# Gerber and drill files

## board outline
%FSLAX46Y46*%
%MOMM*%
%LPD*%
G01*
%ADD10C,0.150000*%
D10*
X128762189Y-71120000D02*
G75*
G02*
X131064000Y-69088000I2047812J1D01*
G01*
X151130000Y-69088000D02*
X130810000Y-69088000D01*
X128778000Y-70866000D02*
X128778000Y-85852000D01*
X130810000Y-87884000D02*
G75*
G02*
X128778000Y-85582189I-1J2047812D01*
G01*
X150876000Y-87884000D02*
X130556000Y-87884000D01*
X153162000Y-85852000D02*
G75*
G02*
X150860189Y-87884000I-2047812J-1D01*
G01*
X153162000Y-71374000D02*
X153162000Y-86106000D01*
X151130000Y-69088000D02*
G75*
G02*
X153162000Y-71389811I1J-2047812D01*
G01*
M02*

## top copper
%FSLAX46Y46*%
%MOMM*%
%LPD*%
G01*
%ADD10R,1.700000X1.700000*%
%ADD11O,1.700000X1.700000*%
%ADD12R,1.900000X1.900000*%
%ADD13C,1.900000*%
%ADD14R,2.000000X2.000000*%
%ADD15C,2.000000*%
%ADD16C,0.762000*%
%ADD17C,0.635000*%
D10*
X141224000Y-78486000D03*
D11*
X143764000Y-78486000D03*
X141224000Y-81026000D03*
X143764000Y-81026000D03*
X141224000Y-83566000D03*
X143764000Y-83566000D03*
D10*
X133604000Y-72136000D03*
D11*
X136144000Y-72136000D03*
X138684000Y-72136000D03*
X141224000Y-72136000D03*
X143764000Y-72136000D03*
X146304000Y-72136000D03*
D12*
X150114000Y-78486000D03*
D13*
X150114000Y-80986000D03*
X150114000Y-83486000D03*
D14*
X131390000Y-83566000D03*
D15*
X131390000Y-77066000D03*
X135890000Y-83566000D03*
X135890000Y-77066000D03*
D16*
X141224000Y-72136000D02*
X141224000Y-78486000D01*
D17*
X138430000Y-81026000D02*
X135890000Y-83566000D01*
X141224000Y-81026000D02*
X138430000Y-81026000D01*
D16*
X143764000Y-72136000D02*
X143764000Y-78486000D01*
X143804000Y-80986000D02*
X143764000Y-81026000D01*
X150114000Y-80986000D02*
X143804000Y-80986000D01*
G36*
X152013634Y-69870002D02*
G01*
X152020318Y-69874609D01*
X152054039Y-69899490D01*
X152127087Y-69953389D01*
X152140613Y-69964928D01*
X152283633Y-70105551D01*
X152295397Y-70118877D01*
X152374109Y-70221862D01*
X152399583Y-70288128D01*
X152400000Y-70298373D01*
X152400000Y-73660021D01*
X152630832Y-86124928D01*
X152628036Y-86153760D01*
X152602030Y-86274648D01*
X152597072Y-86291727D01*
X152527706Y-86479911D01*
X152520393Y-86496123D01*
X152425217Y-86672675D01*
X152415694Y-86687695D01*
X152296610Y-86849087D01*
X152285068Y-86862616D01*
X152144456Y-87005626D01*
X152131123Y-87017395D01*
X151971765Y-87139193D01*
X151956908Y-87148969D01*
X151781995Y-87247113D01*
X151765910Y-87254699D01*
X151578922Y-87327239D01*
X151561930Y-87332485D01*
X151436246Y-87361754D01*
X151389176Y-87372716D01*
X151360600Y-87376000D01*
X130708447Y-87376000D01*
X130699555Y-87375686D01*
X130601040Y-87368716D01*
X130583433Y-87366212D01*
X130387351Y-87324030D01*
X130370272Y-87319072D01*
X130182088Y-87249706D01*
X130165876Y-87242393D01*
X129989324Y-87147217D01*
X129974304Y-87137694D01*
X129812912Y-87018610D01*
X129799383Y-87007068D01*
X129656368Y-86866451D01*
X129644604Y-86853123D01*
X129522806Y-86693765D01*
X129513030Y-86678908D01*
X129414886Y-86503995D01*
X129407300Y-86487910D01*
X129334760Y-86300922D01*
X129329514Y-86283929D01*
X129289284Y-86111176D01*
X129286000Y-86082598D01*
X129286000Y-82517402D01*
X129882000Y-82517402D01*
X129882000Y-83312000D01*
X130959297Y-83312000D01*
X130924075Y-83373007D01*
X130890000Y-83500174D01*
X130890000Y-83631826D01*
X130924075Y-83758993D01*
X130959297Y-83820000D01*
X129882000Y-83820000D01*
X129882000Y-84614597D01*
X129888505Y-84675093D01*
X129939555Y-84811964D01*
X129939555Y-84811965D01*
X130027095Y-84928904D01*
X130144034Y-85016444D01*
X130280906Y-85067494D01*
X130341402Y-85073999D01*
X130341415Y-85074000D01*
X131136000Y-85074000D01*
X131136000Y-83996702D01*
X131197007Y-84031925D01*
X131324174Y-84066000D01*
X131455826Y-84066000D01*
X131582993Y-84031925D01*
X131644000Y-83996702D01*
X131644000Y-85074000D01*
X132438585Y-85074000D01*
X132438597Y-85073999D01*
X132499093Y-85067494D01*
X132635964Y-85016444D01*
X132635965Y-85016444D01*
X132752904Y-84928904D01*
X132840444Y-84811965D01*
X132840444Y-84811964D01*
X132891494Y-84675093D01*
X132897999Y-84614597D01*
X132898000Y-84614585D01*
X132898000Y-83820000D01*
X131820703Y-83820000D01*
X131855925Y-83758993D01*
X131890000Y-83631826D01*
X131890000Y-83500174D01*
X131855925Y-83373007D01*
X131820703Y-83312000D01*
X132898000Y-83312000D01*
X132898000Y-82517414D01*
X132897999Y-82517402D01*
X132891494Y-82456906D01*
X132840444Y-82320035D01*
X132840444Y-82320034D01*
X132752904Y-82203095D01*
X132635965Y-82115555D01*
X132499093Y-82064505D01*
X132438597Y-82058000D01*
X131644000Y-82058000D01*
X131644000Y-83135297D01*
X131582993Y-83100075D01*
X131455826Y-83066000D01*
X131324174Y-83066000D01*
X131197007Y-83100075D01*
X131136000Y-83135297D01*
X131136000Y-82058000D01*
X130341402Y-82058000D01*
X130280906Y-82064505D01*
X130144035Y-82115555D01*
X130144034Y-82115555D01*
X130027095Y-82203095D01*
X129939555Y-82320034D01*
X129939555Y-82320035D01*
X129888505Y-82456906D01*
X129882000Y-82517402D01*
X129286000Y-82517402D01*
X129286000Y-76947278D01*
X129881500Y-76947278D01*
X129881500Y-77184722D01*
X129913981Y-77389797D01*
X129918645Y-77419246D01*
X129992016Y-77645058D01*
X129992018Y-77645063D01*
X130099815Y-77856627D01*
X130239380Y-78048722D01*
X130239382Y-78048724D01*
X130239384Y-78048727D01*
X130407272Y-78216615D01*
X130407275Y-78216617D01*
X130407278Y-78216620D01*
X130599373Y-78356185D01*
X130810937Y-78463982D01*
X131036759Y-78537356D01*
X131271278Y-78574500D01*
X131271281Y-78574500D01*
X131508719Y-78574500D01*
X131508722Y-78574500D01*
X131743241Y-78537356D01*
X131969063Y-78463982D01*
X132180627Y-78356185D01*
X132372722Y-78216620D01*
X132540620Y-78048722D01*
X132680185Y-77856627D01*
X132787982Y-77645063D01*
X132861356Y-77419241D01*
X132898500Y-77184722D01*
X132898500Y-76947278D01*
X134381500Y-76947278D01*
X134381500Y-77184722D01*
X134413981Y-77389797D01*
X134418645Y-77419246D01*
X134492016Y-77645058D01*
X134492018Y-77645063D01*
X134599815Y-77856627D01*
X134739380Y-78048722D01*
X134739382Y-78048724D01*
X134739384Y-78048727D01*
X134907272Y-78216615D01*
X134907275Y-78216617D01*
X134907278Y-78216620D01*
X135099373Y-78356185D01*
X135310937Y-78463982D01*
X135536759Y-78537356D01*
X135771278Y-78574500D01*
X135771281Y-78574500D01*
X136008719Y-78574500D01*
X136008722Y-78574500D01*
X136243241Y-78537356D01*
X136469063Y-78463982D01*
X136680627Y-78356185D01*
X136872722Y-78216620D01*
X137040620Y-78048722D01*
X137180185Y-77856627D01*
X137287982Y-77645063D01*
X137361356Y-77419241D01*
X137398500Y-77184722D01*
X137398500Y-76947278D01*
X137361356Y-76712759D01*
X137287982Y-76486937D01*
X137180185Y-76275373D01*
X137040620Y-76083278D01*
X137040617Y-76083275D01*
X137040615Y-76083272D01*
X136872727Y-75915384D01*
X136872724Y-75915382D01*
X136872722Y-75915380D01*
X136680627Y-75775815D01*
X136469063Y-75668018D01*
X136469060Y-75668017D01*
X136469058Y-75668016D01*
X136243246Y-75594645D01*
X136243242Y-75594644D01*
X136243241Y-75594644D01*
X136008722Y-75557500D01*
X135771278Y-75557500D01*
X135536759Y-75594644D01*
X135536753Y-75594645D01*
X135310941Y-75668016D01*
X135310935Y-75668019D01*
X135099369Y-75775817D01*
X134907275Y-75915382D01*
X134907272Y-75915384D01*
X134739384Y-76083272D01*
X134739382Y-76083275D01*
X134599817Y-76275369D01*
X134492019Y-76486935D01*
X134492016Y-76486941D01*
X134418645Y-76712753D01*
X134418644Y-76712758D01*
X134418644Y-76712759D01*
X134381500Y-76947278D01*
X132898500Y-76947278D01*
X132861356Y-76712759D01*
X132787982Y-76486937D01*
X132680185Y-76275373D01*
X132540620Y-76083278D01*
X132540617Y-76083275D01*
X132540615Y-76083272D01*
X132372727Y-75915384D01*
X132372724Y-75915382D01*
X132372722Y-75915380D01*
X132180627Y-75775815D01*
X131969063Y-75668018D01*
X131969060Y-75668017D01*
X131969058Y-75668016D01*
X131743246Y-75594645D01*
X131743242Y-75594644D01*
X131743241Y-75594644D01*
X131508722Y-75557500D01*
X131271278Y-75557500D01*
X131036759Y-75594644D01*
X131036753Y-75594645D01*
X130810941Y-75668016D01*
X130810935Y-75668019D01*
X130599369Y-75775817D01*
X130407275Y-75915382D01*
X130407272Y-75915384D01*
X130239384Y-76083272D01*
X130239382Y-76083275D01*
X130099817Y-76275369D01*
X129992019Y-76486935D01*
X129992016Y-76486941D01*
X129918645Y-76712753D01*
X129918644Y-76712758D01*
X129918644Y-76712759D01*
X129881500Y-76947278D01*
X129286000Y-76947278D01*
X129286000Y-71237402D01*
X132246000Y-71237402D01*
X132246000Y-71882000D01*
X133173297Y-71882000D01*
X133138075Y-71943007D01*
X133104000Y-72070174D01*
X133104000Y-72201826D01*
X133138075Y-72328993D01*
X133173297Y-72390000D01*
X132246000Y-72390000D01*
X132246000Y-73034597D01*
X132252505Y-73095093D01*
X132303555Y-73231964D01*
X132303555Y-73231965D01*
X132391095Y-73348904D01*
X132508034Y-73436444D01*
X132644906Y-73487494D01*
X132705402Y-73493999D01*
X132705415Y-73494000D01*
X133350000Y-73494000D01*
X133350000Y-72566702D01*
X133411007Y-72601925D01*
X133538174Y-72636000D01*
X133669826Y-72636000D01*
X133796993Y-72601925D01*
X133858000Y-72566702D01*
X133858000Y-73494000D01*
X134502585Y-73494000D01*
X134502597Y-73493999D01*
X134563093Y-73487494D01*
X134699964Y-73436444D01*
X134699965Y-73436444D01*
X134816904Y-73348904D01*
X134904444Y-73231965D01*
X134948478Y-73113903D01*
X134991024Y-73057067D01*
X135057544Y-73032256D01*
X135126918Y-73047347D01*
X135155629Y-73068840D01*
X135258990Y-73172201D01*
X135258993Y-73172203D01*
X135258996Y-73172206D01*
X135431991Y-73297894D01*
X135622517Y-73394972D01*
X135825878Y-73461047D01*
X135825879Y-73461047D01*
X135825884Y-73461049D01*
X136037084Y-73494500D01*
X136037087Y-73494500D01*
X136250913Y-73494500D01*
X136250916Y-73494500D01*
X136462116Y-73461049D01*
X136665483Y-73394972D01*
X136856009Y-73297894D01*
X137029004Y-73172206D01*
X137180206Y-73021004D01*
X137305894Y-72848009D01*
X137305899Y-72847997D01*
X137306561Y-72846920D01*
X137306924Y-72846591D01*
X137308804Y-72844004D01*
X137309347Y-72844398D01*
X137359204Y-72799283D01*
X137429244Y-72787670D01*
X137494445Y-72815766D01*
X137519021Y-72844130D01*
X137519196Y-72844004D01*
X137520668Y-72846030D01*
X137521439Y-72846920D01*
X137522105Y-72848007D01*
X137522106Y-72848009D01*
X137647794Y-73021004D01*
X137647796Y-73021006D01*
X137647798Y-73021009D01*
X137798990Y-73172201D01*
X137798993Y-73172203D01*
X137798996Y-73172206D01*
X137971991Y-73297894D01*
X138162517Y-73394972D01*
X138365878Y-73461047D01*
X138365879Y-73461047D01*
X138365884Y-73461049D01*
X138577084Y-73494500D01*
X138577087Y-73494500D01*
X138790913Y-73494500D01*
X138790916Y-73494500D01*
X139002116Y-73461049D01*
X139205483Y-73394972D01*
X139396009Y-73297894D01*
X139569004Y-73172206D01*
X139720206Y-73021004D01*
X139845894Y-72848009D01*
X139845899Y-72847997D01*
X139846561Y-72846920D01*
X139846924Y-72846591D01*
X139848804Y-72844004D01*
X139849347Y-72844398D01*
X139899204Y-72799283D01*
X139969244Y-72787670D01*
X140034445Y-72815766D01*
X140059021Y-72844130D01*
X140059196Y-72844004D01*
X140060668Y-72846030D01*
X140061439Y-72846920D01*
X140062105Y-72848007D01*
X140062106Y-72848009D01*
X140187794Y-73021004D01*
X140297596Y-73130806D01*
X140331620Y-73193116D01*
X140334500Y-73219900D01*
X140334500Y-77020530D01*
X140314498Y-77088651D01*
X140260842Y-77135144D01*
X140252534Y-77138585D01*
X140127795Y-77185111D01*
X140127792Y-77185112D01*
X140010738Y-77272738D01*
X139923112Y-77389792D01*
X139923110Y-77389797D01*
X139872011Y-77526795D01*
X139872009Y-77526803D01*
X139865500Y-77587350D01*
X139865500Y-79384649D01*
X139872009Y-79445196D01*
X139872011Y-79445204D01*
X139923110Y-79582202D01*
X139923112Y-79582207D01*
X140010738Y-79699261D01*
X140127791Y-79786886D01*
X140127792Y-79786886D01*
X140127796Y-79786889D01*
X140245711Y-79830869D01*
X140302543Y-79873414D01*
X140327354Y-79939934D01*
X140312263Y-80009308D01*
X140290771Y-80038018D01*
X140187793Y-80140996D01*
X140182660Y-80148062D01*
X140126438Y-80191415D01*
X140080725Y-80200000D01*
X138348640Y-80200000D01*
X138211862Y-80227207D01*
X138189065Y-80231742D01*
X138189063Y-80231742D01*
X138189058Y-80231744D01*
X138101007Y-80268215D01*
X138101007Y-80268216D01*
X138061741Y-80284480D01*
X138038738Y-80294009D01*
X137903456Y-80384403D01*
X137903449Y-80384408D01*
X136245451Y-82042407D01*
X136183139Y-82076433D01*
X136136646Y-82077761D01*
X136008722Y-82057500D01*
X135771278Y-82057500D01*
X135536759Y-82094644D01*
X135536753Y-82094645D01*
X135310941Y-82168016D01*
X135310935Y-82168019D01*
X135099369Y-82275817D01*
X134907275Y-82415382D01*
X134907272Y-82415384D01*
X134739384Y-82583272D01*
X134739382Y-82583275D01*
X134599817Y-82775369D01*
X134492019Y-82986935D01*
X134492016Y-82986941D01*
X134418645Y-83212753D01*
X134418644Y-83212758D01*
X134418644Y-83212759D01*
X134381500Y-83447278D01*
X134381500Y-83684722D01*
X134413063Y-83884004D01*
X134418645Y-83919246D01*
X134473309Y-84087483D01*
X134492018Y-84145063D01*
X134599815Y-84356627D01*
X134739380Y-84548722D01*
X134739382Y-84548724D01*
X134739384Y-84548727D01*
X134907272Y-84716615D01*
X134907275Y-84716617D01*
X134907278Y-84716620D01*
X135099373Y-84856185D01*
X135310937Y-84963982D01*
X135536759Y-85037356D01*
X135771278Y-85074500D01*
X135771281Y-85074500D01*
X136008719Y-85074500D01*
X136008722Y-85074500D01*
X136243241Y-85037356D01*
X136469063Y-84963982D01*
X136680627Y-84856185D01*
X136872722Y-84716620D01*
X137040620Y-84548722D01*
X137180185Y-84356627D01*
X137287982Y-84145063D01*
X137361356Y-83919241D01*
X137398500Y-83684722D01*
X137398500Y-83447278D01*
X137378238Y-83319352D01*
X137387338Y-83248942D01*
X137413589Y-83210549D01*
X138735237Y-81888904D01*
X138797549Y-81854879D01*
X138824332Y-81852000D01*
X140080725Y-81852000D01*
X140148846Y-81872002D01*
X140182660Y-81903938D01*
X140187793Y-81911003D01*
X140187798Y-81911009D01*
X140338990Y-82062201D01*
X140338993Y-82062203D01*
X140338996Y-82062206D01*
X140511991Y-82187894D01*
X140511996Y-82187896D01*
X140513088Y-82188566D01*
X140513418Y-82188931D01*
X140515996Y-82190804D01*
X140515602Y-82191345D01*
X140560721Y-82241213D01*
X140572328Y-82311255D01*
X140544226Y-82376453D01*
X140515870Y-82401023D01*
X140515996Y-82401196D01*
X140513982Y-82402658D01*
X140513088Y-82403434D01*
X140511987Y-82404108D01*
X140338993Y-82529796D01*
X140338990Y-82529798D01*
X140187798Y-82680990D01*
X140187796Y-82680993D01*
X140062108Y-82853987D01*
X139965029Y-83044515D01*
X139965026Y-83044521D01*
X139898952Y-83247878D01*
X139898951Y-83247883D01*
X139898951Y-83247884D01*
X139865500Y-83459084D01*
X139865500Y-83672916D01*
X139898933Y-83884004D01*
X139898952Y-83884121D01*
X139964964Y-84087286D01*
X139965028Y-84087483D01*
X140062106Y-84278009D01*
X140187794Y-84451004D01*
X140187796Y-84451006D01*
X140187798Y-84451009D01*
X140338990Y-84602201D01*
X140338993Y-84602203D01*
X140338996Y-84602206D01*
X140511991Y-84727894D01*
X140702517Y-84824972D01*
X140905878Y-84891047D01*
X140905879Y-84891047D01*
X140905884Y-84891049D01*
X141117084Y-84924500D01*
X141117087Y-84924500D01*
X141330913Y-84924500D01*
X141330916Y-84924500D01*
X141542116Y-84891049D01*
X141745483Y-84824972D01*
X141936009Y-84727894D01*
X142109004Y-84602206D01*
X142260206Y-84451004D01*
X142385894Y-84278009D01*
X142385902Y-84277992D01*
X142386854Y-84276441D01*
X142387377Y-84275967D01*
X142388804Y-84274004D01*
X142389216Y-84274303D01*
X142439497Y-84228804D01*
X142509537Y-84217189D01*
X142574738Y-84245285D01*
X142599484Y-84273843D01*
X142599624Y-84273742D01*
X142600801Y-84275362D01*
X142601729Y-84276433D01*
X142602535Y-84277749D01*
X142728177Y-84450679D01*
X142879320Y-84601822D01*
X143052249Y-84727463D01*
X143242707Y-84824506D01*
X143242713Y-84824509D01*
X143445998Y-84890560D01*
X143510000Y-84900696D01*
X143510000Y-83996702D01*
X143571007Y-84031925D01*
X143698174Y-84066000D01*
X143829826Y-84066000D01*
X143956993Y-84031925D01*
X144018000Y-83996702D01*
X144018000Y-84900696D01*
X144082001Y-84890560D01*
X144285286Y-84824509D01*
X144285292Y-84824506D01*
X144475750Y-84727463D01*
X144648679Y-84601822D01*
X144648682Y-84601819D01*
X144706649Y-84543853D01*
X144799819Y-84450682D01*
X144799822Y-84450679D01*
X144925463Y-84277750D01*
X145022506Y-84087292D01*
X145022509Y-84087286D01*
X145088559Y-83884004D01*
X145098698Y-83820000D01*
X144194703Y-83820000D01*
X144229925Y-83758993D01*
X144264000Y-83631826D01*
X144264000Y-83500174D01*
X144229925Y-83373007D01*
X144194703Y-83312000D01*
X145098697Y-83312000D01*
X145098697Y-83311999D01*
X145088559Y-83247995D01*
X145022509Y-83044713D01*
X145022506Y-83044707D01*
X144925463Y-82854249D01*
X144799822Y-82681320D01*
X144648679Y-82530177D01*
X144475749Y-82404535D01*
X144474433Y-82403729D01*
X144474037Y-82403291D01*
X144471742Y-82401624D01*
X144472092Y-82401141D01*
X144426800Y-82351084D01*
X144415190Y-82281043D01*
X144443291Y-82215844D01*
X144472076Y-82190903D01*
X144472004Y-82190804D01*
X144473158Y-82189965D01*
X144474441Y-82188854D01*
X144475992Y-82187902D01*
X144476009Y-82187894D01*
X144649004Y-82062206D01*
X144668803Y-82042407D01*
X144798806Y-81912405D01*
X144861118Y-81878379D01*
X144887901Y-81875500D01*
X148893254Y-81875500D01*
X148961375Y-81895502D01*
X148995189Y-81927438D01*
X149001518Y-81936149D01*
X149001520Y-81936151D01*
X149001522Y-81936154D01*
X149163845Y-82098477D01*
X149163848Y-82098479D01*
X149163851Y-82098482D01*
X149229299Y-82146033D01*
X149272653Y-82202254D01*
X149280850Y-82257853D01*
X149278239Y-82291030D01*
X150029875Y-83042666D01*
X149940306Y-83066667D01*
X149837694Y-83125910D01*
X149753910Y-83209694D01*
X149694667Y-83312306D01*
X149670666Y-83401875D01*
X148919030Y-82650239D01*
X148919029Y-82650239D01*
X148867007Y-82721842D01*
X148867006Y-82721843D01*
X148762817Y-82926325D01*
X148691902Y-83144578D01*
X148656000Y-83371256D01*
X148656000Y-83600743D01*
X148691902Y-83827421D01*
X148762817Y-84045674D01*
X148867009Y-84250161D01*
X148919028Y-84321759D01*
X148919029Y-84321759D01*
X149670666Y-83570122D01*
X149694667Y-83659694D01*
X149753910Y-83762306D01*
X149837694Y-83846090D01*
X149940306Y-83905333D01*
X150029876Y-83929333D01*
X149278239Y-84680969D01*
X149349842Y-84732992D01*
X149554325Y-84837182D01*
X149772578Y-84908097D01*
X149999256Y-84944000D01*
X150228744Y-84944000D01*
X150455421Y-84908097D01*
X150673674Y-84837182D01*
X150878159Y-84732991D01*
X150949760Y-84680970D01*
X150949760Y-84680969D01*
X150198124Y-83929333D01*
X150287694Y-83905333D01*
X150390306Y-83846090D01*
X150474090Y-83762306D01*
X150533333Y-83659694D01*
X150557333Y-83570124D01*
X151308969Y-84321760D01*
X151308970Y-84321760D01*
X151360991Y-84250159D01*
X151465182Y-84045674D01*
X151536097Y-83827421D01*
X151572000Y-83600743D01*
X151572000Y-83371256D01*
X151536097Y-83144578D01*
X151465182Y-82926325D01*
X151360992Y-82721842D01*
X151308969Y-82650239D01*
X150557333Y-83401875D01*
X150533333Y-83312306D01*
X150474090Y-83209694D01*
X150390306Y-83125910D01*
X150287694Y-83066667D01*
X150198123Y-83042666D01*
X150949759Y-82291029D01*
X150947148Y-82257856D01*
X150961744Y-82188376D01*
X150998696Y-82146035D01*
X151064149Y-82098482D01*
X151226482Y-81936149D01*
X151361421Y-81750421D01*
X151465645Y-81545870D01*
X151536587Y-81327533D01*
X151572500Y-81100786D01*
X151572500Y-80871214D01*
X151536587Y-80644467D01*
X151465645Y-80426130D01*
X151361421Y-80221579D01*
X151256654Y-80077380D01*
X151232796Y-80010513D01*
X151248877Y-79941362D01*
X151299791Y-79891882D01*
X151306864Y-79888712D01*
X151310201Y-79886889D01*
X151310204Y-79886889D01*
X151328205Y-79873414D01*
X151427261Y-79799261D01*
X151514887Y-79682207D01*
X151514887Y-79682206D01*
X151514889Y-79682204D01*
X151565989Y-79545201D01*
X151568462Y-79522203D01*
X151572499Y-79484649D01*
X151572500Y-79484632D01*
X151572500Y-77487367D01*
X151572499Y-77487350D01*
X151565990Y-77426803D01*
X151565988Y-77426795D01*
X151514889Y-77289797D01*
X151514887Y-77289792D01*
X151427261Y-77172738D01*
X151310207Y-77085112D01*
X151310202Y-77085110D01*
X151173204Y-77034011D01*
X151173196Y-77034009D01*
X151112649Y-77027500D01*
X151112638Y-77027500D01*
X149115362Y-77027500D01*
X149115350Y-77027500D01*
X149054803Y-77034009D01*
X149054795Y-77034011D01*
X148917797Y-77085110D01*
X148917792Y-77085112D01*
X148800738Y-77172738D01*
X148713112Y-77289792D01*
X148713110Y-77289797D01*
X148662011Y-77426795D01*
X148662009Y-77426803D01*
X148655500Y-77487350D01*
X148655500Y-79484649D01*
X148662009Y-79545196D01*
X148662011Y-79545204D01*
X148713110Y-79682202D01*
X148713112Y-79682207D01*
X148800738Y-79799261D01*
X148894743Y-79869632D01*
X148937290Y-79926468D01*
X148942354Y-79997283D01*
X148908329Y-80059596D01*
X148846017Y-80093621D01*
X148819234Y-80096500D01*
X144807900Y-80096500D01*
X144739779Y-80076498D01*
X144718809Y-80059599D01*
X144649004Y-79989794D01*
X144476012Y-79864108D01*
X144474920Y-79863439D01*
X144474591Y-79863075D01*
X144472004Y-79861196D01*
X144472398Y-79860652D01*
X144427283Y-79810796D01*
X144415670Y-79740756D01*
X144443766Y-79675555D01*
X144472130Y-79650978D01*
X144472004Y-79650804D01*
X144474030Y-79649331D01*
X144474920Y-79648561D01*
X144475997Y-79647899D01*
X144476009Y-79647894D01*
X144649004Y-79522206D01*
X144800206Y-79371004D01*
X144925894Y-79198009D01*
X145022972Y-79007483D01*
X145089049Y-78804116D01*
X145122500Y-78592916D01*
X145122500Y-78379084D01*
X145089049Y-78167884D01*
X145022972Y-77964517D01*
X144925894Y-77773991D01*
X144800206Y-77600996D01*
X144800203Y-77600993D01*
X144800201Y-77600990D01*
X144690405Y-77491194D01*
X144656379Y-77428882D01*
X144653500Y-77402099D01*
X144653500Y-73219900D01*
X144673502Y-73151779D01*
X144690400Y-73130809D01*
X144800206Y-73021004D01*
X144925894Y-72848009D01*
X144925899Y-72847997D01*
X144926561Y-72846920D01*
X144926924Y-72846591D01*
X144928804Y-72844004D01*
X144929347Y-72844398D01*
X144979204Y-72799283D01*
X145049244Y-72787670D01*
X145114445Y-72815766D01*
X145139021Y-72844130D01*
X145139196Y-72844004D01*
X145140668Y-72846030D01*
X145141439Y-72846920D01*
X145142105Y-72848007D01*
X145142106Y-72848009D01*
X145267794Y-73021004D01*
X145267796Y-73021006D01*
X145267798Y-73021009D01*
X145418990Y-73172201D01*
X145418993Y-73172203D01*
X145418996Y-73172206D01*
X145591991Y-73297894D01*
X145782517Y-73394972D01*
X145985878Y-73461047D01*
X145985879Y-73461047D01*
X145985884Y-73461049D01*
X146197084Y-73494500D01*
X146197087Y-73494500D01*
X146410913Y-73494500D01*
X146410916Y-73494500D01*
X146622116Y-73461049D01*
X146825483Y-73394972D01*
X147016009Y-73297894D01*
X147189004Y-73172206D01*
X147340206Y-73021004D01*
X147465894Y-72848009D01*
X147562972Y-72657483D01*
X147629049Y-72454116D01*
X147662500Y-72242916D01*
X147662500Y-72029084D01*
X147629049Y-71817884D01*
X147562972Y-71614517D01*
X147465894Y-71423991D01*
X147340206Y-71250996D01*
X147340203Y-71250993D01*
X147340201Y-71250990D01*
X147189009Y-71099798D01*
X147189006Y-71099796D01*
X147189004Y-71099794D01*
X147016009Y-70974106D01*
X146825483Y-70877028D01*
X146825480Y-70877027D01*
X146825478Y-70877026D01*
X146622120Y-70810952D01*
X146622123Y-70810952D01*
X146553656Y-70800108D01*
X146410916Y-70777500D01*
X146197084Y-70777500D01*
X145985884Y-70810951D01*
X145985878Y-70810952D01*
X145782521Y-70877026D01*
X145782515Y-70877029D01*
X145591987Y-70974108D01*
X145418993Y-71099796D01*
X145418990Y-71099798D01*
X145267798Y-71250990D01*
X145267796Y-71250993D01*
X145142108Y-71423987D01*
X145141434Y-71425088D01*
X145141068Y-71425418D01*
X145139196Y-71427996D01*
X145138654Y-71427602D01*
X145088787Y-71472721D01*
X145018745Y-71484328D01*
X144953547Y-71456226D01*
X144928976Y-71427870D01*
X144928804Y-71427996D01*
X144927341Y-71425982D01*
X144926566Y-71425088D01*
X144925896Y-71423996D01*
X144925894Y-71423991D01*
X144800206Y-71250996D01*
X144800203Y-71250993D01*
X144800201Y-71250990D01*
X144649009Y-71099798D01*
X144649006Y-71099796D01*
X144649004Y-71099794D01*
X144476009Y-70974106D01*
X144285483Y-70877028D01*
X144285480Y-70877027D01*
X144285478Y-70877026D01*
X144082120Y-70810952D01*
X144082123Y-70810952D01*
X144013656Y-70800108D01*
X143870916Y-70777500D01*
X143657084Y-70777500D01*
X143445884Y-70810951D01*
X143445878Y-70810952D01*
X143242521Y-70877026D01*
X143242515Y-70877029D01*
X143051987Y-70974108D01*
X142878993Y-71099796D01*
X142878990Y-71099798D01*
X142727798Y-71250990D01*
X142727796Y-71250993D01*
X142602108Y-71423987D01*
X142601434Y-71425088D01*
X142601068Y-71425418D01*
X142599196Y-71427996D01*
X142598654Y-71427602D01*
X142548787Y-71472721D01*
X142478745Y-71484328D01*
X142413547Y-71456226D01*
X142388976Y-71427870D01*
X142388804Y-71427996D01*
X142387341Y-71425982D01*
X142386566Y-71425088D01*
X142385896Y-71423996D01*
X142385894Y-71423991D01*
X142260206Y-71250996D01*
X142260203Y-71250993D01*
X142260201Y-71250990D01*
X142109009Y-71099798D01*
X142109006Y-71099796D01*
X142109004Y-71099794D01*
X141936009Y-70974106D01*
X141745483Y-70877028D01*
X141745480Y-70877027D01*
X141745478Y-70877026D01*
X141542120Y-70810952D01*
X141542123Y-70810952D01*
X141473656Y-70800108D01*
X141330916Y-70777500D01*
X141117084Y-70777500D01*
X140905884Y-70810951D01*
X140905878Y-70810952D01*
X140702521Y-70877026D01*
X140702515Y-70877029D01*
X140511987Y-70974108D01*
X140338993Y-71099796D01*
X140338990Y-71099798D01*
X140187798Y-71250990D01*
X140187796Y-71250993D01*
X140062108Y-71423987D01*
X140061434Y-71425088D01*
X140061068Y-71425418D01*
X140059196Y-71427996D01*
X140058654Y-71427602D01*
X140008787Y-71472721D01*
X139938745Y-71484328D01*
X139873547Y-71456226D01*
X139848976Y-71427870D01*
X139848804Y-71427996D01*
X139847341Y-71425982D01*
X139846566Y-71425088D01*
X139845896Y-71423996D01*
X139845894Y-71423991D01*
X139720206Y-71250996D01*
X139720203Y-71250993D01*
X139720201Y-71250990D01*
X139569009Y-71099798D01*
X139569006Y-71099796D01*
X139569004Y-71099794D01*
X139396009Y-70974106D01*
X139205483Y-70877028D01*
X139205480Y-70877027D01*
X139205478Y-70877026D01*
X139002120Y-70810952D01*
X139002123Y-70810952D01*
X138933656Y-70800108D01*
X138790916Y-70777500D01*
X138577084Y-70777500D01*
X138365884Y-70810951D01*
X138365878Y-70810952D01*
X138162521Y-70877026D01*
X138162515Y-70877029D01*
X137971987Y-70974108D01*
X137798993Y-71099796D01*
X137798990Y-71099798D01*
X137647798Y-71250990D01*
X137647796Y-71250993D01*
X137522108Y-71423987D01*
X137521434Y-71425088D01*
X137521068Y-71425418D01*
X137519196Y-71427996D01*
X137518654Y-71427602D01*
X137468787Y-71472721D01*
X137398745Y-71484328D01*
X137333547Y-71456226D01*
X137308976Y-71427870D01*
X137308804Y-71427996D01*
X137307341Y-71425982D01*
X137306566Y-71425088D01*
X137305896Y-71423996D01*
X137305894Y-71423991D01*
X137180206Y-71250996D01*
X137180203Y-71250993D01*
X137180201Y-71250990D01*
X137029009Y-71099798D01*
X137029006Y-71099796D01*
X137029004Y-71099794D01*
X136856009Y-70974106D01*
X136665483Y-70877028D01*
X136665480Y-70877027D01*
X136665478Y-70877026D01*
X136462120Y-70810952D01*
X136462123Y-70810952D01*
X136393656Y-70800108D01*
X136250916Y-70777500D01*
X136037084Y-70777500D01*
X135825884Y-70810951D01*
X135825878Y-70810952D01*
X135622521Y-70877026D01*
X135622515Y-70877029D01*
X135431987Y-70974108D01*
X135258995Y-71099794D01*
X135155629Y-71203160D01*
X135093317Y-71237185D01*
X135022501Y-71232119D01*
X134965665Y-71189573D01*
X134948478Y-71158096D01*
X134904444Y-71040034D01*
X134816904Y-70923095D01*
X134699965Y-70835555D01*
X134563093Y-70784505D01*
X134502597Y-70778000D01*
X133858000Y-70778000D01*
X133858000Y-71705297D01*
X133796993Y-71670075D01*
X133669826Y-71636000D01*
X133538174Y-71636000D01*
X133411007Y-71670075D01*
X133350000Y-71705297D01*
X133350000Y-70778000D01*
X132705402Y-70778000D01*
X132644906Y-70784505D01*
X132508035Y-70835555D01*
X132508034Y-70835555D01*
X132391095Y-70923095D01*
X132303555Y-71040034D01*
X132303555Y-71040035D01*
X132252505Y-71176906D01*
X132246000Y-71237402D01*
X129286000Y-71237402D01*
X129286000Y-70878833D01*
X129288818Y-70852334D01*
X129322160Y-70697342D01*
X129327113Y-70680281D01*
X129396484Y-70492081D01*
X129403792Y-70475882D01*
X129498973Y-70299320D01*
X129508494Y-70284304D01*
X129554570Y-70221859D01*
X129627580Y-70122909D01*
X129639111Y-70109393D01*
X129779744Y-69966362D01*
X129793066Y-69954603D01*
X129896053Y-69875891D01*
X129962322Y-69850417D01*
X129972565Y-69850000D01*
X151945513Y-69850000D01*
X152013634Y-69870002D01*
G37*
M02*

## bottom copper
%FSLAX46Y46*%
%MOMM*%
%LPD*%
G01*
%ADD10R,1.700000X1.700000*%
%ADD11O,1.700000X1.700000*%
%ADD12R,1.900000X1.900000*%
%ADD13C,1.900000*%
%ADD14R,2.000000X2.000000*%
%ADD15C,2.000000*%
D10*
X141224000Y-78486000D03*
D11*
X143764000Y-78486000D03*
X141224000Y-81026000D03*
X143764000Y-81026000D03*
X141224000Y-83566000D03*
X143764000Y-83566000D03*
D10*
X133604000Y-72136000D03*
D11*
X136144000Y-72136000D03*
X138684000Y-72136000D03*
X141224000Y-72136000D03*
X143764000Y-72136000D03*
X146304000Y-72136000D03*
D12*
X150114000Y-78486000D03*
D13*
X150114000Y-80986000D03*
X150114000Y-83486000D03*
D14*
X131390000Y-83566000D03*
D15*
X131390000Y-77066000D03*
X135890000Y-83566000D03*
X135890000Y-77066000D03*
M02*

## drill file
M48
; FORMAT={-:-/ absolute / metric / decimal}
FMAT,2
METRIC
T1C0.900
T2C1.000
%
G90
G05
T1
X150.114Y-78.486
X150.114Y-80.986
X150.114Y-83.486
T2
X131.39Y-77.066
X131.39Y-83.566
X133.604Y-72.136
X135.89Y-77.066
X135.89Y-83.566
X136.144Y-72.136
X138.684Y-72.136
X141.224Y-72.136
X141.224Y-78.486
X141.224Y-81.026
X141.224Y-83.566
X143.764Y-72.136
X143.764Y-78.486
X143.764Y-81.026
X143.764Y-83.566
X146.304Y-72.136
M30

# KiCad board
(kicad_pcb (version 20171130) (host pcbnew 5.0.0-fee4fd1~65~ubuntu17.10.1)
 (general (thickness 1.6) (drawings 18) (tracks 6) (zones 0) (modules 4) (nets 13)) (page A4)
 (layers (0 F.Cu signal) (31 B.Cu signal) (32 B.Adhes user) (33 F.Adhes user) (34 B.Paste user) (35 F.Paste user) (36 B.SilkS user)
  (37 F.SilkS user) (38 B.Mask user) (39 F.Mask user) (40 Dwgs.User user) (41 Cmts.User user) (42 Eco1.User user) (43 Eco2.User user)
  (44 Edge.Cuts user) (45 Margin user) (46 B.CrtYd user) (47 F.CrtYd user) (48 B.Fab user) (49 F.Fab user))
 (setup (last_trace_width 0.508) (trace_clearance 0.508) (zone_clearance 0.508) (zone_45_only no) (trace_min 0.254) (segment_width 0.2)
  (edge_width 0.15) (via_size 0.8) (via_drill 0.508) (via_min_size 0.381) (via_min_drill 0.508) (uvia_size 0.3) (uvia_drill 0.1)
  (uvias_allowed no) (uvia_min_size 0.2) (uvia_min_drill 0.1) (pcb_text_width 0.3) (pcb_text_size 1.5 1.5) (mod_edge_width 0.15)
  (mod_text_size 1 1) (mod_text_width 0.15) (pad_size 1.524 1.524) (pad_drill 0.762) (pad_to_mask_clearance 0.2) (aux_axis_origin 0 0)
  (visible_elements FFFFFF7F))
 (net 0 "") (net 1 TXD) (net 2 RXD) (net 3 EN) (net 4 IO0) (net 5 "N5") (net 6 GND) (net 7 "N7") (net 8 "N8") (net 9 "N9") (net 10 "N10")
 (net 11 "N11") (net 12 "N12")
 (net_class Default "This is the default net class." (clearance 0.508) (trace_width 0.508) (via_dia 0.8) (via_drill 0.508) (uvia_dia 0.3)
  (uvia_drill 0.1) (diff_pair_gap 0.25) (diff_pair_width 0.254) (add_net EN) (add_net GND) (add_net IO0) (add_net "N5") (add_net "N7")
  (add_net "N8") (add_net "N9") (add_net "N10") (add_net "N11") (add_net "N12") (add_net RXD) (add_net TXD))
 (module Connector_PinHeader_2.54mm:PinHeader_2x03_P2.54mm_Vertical (layer F.Cu) (at 141.224 78.486)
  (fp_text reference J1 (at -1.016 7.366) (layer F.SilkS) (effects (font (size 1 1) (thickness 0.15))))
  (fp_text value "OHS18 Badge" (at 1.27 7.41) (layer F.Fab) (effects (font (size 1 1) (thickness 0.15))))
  (pad 1 thru_hole rect (at 0 0) (size 1.7 1.7) (drill 1) (layers *.Cu *.Mask) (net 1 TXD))
  (pad 2 thru_hole oval (at 2.54 0) (size 1.7 1.7) (drill 1) (layers *.Cu *.Mask) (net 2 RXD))
  (pad 3 thru_hole oval (at 0 2.54) (size 1.7 1.7) (drill 1) (layers *.Cu *.Mask) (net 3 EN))
  (pad 4 thru_hole oval (at 2.54 2.54) (size 1.7 1.7) (drill 1) (layers *.Cu *.Mask) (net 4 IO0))
  (pad 5 thru_hole oval (at 0 5.08) (size 1.7 1.7) (drill 1) (layers *.Cu *.Mask) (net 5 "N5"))
  (pad 6 thru_hole oval (at 2.54 5.08) (size 1.7 1.7) (drill 1) (layers *.Cu *.Mask) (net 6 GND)))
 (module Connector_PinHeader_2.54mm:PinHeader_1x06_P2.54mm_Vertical (layer F.Cu) (at 133.604 72.136 90)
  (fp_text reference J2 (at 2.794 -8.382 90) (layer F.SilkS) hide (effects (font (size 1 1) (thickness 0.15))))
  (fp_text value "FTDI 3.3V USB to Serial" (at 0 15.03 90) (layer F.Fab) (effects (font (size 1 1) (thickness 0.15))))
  (pad 1 thru_hole rect (at 0 0 90) (size 1.7 1.7) (drill 1) (layers *.Cu *.Mask) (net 6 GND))
  (pad 2 thru_hole oval (at 0 2.54 90) (size 1.7 1.7) (drill 1) (layers *.Cu *.Mask) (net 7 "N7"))
  (pad 3 thru_hole oval (at 0 5.08 90) (size 1.7 1.7) (drill 1) (layers *.Cu *.Mask) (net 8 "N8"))
  (pad 4 thru_hole oval (at 0 7.62 90) (size 1.7 1.7) (drill 1) (layers *.Cu *.Mask) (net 1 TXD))
  (pad 5 thru_hole oval (at 0 10.16 90) (size 1.7 1.7) (drill 1) (layers *.Cu *.Mask) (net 2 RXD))
  (pad 6 thru_hole oval (at 0 12.7 90) (size 1.7 1.7) (drill 1) (layers *.Cu *.Mask) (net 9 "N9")))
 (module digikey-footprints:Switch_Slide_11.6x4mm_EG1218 (layer F.Cu) (at 150.114 78.486 270)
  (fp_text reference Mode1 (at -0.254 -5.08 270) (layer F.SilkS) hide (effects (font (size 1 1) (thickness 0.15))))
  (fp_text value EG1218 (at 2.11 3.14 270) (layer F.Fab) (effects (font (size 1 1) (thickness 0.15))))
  (pad 1 thru_hole rect (at 0 0 270) (size 1.9 1.9) (drill 0.9) (layers *.Cu *.Mask) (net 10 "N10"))
  (pad 2 thru_hole circle (at 2.5 0 270) (size 1.9 1.9) (drill 0.9) (layers *.Cu *.Mask) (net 4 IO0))
  (pad 3 thru_hole circle (at 5 0 270) (size 1.9 1.9) (drill 0.9) (layers *.Cu *.Mask) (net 6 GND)))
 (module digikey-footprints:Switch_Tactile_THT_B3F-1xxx (layer F.Cu) (at 131.3794 83.5672 90)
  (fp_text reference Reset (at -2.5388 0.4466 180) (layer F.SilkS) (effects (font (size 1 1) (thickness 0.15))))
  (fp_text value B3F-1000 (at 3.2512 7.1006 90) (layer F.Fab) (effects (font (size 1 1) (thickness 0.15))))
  (pad 1 thru_hole rect (at 0.0012 0.0106 90) (size 2 2) (drill 1) (layers *.Cu *.Mask) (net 6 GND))
  (pad 2 thru_hole circle (at 6.5012 0.0106 90) (size 2 2) (drill 1) (layers *.Cu *.Mask) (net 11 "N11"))
  (pad 3 thru_hole circle (at 0.0012 4.5106 90) (size 2 2) (drill 1) (layers *.Cu *.Mask) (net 3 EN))
  (pad 4 thru_hole circle (at 6.5012 4.5106 90) (size 2 2) (drill 1) (layers *.Cu *.Mask) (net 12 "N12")))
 (gr_arc (start 130.810001 71.119999) (end 131.064 69.088) (angle -97.12501635) (layer Edge.Cuts) (width 0.15))
 (gr_line (start 151.13 69.088) (end 130.81 69.088) (layer Edge.Cuts) (width 0.15))
 (gr_line (start 128.778 70.866) (end 128.778 85.852) (layer Edge.Cuts) (width 0.15))
 (gr_arc (start 130.809999 85.836188) (end 128.778 85.582189) (angle -97.12501635) (layer Edge.Cuts) (width 0.15))
 (gr_line (start 150.876 87.884) (end 130.556 87.884) (layer Edge.Cuts) (width 0.15))
 (gr_arc (start 151.114188 85.852001) (end 150.860189 87.884) (angle -97.12501635) (layer Edge.Cuts) (width 0.15))
 (gr_line (start 153.162 71.374) (end 153.162 86.106) (layer Edge.Cuts) (width 0.15))
 (gr_arc (start 151.130001 71.135812) (end 153.162 71.389811) (angle -97.12501635) (layer Edge.Cuts) (width 0.15))
 (segment (start 141.224 72.136) (end 141.224 78.486) (width 0.762) (layer F.Cu) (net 1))
 (segment (start 138.43 81.026) (end 135.89 83.566) (width 0.635) (layer F.Cu) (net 3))
 (segment (start 141.224 81.026) (end 138.43 81.026) (width 0.635) (layer F.Cu) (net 3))
 (segment (start 143.764 72.136) (end 143.764 78.486) (width 0.762) (layer F.Cu) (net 2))
 (segment (start 143.804 80.986) (end 143.764 81.026) (width 0.762) (layer F.Cu) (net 4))
 (segment (start 150.114 80.986) (end 143.804 80.986) (width 0.762) (layer F.Cu) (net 4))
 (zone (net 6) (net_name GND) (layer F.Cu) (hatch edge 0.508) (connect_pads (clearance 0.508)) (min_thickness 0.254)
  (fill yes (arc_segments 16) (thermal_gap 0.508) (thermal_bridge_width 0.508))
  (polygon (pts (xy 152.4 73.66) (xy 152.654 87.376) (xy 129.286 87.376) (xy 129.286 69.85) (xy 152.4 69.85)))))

